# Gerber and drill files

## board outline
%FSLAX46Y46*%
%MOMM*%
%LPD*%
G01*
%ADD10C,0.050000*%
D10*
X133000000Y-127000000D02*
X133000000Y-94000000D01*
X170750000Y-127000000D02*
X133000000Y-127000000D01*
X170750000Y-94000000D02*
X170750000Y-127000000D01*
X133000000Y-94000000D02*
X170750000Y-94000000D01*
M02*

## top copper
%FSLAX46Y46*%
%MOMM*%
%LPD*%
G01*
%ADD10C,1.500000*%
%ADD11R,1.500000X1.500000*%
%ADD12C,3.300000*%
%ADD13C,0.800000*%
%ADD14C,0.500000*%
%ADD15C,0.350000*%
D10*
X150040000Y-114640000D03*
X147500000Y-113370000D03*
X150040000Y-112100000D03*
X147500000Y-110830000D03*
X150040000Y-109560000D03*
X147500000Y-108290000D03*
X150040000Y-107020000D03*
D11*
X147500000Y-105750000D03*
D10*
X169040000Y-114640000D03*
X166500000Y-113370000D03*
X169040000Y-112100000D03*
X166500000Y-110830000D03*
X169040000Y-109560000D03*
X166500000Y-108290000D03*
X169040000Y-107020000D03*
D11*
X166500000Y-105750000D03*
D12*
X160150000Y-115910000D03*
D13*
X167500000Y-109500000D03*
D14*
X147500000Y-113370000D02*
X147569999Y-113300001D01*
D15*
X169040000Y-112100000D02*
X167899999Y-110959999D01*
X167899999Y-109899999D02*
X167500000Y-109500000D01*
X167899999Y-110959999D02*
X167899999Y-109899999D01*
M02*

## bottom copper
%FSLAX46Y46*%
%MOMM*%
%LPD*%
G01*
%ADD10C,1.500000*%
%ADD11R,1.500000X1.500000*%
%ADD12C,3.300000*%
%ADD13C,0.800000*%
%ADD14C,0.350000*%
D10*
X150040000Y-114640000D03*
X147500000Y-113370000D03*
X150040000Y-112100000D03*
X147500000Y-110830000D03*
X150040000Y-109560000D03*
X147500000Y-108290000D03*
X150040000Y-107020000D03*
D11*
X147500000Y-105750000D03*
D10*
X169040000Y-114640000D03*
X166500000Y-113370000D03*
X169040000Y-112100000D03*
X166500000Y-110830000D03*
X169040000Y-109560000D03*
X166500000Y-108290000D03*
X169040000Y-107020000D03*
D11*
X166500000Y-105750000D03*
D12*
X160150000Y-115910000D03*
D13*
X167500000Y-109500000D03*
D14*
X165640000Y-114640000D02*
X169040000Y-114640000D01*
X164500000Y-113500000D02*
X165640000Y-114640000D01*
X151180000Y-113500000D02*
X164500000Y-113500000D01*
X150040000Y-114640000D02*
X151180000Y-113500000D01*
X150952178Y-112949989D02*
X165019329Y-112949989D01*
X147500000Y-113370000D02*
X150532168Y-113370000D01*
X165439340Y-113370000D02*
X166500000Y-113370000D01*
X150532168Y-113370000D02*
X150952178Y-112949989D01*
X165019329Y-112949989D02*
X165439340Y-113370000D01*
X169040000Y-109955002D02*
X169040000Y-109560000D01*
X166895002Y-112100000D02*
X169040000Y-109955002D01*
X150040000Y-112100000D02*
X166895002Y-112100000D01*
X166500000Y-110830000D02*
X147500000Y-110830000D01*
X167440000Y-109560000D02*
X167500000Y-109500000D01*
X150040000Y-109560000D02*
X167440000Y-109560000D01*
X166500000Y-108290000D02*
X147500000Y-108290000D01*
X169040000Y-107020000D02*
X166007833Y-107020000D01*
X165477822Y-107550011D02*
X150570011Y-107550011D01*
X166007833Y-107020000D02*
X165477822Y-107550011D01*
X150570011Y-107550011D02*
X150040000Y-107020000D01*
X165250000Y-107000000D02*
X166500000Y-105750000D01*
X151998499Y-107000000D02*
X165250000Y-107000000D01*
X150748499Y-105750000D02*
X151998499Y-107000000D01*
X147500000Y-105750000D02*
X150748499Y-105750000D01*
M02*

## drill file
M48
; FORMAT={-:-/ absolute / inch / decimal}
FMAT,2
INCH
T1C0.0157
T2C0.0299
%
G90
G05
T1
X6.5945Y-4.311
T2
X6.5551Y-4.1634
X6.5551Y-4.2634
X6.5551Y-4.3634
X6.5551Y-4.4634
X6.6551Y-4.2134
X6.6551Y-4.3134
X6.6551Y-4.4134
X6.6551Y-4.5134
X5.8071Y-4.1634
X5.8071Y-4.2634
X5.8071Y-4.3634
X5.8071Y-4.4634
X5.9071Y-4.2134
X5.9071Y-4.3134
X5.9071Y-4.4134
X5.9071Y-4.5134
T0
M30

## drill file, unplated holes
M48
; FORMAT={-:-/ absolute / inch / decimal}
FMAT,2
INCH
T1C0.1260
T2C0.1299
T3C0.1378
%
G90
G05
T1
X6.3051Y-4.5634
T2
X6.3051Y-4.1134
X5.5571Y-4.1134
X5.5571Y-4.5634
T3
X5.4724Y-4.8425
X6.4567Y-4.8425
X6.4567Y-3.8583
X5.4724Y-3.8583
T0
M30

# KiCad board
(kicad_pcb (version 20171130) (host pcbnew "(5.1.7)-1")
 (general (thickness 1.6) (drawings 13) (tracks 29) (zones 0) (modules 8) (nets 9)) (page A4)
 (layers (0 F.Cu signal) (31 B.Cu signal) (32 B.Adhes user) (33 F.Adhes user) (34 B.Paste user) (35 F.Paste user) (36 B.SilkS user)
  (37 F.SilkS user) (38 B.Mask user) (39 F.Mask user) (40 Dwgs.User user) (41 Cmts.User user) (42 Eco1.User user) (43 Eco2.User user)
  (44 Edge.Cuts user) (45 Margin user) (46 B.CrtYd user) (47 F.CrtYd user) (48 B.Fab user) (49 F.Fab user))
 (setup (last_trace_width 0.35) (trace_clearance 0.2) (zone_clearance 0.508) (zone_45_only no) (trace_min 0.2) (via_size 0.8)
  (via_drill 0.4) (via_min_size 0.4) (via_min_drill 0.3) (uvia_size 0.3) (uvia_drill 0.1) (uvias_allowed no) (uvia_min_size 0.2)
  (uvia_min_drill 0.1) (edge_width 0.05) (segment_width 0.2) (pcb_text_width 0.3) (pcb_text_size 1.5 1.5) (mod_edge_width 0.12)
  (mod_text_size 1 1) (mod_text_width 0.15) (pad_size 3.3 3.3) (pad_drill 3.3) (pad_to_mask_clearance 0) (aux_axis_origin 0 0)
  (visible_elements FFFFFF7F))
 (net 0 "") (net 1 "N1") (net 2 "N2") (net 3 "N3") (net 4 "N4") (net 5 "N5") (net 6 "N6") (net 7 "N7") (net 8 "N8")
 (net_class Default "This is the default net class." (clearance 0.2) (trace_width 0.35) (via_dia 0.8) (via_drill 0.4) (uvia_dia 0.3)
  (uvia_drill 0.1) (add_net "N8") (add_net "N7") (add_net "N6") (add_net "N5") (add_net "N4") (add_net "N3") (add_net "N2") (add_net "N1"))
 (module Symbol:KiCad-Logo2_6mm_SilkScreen (layer B.Cu) (at 151.5 121.5 180)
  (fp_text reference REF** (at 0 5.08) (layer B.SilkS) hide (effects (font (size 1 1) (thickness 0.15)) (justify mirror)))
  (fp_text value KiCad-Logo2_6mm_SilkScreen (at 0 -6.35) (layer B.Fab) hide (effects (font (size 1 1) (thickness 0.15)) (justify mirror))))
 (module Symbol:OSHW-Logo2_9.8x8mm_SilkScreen (layer B.Cu) (at 151 98.5 180)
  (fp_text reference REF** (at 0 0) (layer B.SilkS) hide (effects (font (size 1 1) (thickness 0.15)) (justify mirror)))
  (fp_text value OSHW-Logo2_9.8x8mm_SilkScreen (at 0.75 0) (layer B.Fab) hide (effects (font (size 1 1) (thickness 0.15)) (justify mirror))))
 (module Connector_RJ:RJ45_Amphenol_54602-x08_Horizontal (layer F.Cu) (at 147.5 105.75 270)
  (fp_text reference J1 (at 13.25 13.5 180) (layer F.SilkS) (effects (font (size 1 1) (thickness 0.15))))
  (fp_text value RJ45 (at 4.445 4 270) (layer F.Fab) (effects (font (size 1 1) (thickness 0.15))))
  (pad 8 thru_hole circle (at 8.89 -2.54 270) (size 1.5 1.5) (drill 0.76) (layers *.Cu *.Mask) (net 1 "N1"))
  (pad 7 thru_hole circle (at 7.62 0 270) (size 1.5 1.5) (drill 0.76) (layers *.Cu *.Mask) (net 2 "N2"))
  (pad 6 thru_hole circle (at 6.35 -2.54 270) (size 1.5 1.5) (drill 0.76) (layers *.Cu *.Mask) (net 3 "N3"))
  (pad 5 thru_hole circle (at 5.08 0 270) (size 1.5 1.5) (drill 0.76) (layers *.Cu *.Mask) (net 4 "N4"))
  (pad 4 thru_hole circle (at 3.81 -2.54 270) (size 1.5 1.5) (drill 0.76) (layers *.Cu *.Mask) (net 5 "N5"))
  (pad 3 thru_hole circle (at 2.54 0 270) (size 1.5 1.5) (drill 0.76) (layers *.Cu *.Mask) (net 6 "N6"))
  (pad 2 thru_hole circle (at 1.27 -2.54 270) (size 1.5 1.5) (drill 0.76) (layers *.Cu *.Mask) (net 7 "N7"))
  (pad 1 thru_hole rect (at 0 0 270) (size 1.5 1.5) (drill 0.76) (layers *.Cu *.Mask) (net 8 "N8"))
  (pad "" np_thru_hole circle (at -1.27 6.35 270) (size 3.3 3.3) (drill 3.3) (layers *.Cu *.Mask))
  (pad "" np_thru_hole circle (at 10.16 6.35 270) (size 3.3 3.3) (drill 3.3) (layers *.Cu *.Mask)))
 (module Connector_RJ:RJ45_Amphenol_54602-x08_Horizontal (layer F.Cu) (at 166.5 105.75 270)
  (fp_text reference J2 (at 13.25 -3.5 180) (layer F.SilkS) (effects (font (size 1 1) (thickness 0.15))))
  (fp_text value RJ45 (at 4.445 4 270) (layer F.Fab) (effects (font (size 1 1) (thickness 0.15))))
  (pad 8 thru_hole circle (at 8.89 -2.54 270) (size 1.5 1.5) (drill 0.76) (layers *.Cu *.Mask) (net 1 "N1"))
  (pad 7 thru_hole circle (at 7.62 0 270) (size 1.5 1.5) (drill 0.76) (layers *.Cu *.Mask) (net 2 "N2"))
  (pad 6 thru_hole circle (at 6.35 -2.54 270) (size 1.5 1.5) (drill 0.76) (layers *.Cu *.Mask) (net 5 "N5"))
  (pad 5 thru_hole circle (at 5.08 0 270) (size 1.5 1.5) (drill 0.76) (layers *.Cu *.Mask) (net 4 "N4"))
  (pad 4 thru_hole circle (at 3.81 -2.54 270) (size 1.5 1.5) (drill 0.76) (layers *.Cu *.Mask) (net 3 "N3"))
  (pad 3 thru_hole circle (at 2.54 0 270) (size 1.5 1.5) (drill 0.76) (layers *.Cu *.Mask) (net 6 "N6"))
  (pad 2 thru_hole circle (at 1.27 -2.54 270) (size 1.5 1.5) (drill 0.76) (layers *.Cu *.Mask) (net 7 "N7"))
  (pad 1 thru_hole rect (at 0 0 270) (size 1.5 1.5) (drill 0.76) (layers *.Cu *.Mask) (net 8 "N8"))
  (pad "" np_thru_hole circle (at -1.27 6.35 270) (size 3.3 3.3) (drill 3.3) (layers *.Cu *.Mask))
  (pad "" np_thru_hole circle (at 10.16 6.35 270) (size 3.3 3.3) (drill 3.2) (layers *.Cu *.Mask)))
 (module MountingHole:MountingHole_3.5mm (layer F.Cu) (at 164 123)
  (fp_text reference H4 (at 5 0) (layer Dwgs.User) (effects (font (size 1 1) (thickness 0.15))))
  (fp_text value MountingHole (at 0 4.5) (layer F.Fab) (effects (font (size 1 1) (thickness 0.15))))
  (pad 1 np_thru_hole circle (at 0 0) (size 3.5 3.5) (drill 3.5) (layers *.Cu *.Mask)))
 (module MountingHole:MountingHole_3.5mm (layer F.Cu) (at 164 98)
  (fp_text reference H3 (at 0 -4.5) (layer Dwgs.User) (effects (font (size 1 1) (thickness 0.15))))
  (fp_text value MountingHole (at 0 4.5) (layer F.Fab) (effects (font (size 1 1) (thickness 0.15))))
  (pad 1 np_thru_hole circle (at 0 0) (size 3.5 3.5) (drill 3.5) (layers *.Cu *.Mask)))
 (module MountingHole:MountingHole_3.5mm (layer F.Cu) (at 139 123)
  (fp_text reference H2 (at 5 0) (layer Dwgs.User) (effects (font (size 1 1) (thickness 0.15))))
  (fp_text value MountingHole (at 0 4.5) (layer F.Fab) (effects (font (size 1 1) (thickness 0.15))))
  (pad 1 np_thru_hole circle (at 0 0) (size 3.5 3.5) (drill 3.5) (layers *.Cu *.Mask)))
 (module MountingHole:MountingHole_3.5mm (layer F.Cu) (at 139 98)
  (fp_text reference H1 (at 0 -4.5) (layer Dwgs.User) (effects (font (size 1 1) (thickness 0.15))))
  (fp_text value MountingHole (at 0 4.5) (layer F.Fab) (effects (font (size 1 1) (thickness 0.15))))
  (pad 1 np_thru_hole circle (at 0 0) (size 3.5 3.5) (drill 3.5) (layers *.Cu *.Mask)))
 (gr_line (start 133 127) (end 133 94) (layer Edge.Cuts) (width 0.05))
 (gr_line (start 170.75 127) (end 133 127) (layer Edge.Cuts) (width 0.05))
 (gr_line (start 170.75 94) (end 170.75 127) (layer Edge.Cuts) (width 0.05))
 (gr_line (start 133 94) (end 170.75 94) (layer Edge.Cuts) (width 0.05))
 (segment (start 165.64 114.64) (end 169.04 114.64) (width 0.35) (layer B.Cu) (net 1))
 (segment (start 164.5 113.5) (end 165.64 114.64) (width 0.35) (layer B.Cu) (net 1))
 (segment (start 151.18 113.5) (end 164.5 113.5) (width 0.35) (layer B.Cu) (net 1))
 (segment (start 150.04 114.64) (end 151.18 113.5) (width 0.35) (layer B.Cu) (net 1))
 (segment (start 147.5 113.37) (end 147.569999 113.300001) (width 0.5) (layer F.Cu) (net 2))
 (segment (start 150.952178 112.949989) (end 165.019329 112.949989) (width 0.35) (layer B.Cu) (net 2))
 (segment (start 147.5 113.37) (end 150.532168 113.37) (width 0.35) (layer B.Cu) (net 2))
 (segment (start 165.43934 113.37) (end 166.5 113.37) (width 0.35) (layer B.Cu) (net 2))
 (segment (start 150.532168 113.37) (end 150.952178 112.949989) (width 0.35) (layer B.Cu) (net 2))
 (segment (start 165.019329 112.949989) (end 165.43934 113.37) (width 0.35) (layer B.Cu) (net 2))
 (segment (start 169.04 109.955002) (end 169.04 109.56) (width 0.35) (layer B.Cu) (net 3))
 (segment (start 166.895002 112.1) (end 169.04 109.955002) (width 0.35) (layer B.Cu) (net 3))
 (segment (start 150.04 112.1) (end 166.895002 112.1) (width 0.35) (layer B.Cu) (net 3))
 (segment (start 166.5 110.83) (end 147.5 110.83) (width 0.35) (layer B.Cu) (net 4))
 (segment (start 169.04 112.1) (end 167.899999 110.959999) (width 0.35) (layer F.Cu) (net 5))
 (segment (start 167.899999 109.899999) (end 167.5 109.5) (width 0.35) (layer F.Cu) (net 5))
 (segment (start 167.44 109.56) (end 167.5 109.5) (width 0.35) (layer B.Cu) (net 5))
 (segment (start 167.899999 110.959999) (end 167.899999 109.899999) (width 0.35) (layer F.Cu) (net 5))
 (segment (start 150.04 109.56) (end 167.44 109.56) (width 0.35) (layer B.Cu) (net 5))
 (via (at 167.5 109.5) (size 0.8) (drill 0.4) (layers F.Cu B.Cu) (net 5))
 (segment (start 166.5 108.29) (end 147.5 108.29) (width 0.35) (layer B.Cu) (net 6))
 (segment (start 169.04 107.02) (end 166.007833 107.02) (width 0.35) (layer B.Cu) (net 7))
 (segment (start 165.477822 107.550011) (end 150.570011 107.550011) (width 0.35) (layer B.Cu) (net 7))
 (segment (start 166.007833 107.02) (end 165.477822 107.550011) (width 0.35) (layer B.Cu) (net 7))
 (segment (start 150.570011 107.550011) (end 150.04 107.02) (width 0.35) (layer B.Cu) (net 7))
 (segment (start 165.25 107) (end 166.5 105.75) (width 0.35) (layer B.Cu) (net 8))
 (segment (start 151.998499 107) (end 165.25 107) (width 0.35) (layer B.Cu) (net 8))
 (segment (start 150.748499 105.75) (end 151.998499 107) (width 0.35) (layer B.Cu) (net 8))
 (segment (start 147.5 105.75) (end 150.748499 105.75) (width 0.35) (layer B.Cu) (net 8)))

